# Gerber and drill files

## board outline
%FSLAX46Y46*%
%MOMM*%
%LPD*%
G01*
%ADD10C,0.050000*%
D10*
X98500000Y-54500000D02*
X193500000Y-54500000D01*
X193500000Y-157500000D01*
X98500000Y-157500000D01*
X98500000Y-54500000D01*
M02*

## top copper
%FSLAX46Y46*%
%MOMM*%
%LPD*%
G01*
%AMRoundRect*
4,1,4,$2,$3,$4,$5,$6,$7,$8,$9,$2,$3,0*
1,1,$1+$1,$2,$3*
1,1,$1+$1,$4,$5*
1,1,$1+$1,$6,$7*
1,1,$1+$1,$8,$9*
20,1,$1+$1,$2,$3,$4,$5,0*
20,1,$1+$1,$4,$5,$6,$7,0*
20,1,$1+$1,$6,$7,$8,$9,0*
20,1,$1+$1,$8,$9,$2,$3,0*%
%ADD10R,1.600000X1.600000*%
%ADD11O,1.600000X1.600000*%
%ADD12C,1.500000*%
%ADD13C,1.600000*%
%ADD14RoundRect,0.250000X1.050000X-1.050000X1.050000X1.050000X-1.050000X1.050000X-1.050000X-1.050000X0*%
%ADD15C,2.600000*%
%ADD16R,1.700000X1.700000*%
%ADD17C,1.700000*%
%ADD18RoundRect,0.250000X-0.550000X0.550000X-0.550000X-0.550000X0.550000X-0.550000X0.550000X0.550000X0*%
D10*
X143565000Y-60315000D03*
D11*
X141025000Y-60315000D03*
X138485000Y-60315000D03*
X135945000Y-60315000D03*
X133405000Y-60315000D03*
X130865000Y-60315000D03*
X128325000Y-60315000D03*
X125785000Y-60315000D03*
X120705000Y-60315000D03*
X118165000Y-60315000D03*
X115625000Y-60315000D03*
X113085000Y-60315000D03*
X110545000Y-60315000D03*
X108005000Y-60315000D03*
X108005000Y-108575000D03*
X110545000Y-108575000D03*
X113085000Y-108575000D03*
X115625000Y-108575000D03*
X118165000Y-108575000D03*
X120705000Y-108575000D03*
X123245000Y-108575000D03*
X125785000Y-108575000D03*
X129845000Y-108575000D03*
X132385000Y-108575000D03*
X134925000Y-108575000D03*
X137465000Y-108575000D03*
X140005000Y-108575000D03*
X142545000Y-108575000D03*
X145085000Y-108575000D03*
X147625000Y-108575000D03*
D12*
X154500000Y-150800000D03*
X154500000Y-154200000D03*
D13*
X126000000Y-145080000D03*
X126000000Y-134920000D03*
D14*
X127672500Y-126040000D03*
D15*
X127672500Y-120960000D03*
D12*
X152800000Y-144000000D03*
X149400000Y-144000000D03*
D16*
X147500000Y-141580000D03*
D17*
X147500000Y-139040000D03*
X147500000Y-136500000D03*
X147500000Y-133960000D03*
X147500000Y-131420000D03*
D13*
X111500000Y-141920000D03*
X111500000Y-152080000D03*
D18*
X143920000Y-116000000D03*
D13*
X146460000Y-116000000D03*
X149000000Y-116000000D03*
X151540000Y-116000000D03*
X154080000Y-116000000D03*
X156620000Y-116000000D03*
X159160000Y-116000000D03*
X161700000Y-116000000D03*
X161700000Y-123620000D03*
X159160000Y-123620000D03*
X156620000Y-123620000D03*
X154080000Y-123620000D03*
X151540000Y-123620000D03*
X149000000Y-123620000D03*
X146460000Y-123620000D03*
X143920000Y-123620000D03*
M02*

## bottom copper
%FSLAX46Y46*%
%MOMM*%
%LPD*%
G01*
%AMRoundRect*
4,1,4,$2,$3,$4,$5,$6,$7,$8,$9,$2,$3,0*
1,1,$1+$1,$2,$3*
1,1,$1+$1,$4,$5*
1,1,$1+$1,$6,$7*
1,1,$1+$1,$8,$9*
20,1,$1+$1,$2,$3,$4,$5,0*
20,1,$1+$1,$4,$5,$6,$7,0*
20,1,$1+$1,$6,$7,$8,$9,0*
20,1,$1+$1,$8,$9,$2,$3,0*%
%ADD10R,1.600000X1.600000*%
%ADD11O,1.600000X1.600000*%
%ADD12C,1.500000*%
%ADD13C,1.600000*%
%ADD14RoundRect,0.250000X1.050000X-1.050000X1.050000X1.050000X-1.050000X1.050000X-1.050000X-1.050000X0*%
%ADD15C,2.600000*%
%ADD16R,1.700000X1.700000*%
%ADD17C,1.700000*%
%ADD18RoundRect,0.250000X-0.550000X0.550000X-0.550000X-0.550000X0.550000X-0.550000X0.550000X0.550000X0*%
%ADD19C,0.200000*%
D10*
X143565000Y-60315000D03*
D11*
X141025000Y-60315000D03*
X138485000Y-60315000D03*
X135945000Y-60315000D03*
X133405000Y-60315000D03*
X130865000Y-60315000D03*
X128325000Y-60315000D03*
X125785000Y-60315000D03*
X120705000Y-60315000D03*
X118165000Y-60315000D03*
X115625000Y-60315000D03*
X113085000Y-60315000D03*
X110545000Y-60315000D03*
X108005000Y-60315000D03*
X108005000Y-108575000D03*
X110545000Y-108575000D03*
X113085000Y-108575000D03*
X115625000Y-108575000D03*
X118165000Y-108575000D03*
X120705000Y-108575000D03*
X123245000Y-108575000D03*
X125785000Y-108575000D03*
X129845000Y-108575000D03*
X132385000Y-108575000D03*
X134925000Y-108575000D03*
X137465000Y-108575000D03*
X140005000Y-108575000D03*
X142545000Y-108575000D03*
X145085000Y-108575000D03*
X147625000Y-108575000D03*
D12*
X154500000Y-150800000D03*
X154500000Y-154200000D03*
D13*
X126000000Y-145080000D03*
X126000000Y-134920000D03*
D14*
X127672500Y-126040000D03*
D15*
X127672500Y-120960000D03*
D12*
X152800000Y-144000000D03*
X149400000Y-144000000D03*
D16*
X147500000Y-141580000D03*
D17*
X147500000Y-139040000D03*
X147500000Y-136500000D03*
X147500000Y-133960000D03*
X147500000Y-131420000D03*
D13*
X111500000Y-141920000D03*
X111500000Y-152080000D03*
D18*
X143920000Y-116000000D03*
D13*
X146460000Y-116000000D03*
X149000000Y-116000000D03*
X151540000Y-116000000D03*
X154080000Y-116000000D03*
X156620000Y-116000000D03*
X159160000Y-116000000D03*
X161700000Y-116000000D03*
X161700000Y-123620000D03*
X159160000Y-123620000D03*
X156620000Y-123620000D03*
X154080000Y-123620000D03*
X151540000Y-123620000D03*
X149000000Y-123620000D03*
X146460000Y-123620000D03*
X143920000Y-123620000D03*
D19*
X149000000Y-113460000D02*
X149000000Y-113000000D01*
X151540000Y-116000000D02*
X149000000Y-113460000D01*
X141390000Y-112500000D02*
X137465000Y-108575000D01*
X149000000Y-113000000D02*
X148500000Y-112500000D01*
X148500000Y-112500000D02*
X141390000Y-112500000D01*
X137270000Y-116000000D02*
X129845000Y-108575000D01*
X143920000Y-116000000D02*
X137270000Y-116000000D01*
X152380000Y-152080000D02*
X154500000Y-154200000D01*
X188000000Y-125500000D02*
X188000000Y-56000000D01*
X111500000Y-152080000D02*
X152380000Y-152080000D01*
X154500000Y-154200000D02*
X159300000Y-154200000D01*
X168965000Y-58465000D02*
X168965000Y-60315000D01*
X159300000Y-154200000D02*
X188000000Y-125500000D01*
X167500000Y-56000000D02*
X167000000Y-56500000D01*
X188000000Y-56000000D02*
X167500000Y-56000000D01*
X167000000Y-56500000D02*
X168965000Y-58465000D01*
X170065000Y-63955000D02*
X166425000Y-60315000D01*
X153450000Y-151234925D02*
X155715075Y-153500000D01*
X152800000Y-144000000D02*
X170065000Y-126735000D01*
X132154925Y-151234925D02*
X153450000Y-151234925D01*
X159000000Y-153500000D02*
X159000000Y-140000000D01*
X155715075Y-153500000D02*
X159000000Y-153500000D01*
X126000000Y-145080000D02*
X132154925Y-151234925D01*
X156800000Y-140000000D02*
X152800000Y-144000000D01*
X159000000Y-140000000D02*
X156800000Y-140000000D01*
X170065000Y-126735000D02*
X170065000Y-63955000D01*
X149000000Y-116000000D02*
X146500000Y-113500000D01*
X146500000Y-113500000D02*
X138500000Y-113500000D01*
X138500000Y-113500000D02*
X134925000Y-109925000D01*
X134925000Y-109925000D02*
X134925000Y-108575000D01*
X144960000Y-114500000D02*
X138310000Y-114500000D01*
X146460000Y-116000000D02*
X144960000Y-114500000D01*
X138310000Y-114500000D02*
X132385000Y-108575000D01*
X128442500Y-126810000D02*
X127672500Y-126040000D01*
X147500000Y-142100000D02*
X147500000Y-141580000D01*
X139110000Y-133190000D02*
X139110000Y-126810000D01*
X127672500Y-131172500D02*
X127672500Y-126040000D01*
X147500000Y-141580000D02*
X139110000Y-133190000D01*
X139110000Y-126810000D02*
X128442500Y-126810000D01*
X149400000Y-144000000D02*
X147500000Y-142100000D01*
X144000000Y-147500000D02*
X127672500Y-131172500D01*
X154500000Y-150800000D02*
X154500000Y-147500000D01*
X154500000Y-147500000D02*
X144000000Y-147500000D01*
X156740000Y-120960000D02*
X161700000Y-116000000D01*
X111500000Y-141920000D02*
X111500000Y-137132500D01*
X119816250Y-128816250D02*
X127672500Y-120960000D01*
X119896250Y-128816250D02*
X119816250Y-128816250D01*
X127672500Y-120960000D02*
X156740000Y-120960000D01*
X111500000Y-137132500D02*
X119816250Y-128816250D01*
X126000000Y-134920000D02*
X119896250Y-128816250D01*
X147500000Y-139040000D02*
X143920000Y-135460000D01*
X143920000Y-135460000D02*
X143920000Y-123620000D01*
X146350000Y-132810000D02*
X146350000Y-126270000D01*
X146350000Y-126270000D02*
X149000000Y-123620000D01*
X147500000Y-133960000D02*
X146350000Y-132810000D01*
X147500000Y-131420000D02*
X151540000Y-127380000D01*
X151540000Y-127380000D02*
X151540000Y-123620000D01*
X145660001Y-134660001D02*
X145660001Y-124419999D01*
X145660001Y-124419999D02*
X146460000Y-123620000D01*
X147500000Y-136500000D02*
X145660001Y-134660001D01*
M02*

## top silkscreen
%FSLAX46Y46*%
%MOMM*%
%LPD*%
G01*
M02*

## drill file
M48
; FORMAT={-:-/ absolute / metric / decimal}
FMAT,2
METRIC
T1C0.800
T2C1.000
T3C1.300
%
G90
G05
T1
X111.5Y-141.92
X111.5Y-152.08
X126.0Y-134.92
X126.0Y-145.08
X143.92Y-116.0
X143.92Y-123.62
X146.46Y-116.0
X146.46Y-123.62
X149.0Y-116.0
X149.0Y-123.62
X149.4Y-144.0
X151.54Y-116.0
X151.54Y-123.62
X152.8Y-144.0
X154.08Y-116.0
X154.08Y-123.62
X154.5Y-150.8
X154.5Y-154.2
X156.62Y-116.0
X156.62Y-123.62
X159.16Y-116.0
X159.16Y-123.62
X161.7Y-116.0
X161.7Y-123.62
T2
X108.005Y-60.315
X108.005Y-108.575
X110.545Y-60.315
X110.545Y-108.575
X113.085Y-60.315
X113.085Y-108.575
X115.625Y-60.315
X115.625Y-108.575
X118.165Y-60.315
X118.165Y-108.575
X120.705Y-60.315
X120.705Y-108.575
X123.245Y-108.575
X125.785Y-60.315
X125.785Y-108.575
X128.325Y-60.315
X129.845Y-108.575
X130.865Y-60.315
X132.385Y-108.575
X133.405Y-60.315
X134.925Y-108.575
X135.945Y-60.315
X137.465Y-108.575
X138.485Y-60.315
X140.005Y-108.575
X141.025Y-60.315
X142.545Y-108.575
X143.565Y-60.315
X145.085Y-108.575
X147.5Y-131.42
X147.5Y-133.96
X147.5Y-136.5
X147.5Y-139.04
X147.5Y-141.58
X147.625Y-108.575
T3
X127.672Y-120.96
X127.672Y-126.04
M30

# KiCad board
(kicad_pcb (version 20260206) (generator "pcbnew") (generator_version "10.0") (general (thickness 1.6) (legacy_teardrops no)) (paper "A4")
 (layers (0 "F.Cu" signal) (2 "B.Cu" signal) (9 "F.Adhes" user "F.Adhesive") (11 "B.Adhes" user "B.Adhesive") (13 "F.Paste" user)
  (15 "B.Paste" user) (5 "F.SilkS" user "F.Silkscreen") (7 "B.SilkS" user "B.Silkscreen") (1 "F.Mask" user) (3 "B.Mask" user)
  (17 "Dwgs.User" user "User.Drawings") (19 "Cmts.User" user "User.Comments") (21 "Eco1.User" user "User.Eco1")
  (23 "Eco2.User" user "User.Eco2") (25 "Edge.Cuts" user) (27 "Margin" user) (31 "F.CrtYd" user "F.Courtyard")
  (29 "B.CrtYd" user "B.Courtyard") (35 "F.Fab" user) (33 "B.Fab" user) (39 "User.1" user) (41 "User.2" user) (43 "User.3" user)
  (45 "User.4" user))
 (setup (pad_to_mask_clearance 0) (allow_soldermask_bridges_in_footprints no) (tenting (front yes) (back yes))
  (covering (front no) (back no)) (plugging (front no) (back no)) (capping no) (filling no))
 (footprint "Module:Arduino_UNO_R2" (layer "B.Cu") (at 143.565 60.315 180)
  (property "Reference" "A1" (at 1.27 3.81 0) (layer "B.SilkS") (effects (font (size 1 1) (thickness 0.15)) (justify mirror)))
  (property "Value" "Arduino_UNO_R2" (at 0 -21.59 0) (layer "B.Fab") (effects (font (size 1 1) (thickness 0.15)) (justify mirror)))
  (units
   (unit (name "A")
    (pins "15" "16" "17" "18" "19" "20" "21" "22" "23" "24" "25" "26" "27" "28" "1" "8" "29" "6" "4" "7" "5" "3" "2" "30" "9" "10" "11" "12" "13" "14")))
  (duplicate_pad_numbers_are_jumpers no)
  (pad "1" thru_hole rect (at 0 0 90) (size 1.6 1.6) (drill 1) (layers "*.Cu" "*.Mask") (remove_unused_layers no)
   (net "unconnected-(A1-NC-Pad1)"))
  (pad "2" thru_hole oval (at 2.54 0 90) (size 1.6 1.6) (drill 1) (layers "*.Cu" "*.Mask") (remove_unused_layers no)
   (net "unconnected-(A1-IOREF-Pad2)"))
  (pad "3" thru_hole oval (at 5.08 0 90) (size 1.6 1.6) (drill 1) (layers "*.Cu" "*.Mask") (remove_unused_layers no)
   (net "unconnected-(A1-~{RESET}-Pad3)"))
  (pad "4" thru_hole oval (at 7.62 0 90) (size 1.6 1.6) (drill 1) (layers "*.Cu" "*.Mask") (remove_unused_layers no)
   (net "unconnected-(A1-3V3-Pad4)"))
  (pad "5" thru_hole oval (at 10.16 0 90) (size 1.6 1.6) (drill 1) (layers "*.Cu" "*.Mask") (remove_unused_layers no)
   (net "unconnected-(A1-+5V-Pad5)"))
  (pad "6" thru_hole oval (at 12.7 0 90) (size 1.6 1.6) (drill 1) (layers "*.Cu" "*.Mask") (remove_unused_layers no)
   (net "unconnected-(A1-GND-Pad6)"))
  (pad "7" thru_hole oval (at 15.24 0 90) (size 1.6 1.6) (drill 1) (layers "*.Cu" "*.Mask") (remove_unused_layers no)
   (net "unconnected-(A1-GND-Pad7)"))
  (pad "8" thru_hole oval (at 17.78 0 90) (size 1.6 1.6) (drill 1) (layers "*.Cu" "*.Mask") (remove_unused_layers no)
   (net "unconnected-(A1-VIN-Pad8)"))
  (pad "9" thru_hole oval (at 22.86 0 90) (size 1.6 1.6) (drill 1) (layers "*.Cu" "*.Mask") (remove_unused_layers no) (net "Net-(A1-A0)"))
  (pad "10" thru_hole oval (at 25.4 0 90) (size 1.6 1.6) (drill 1) (layers "*.Cu" "*.Mask") (remove_unused_layers no) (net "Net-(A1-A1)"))
  (pad "11" thru_hole oval (at 27.94 0 90) (size 1.6 1.6) (drill 1) (layers "*.Cu" "*.Mask") (remove_unused_layers no)
   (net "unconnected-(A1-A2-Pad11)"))
  (pad "12" thru_hole oval (at 30.48 0 90) (size 1.6 1.6) (drill 1) (layers "*.Cu" "*.Mask") (remove_unused_layers no)
   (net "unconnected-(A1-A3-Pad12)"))
  (pad "13" thru_hole oval (at 33.02 0 90) (size 1.6 1.6) (drill 1) (layers "*.Cu" "*.Mask") (remove_unused_layers no)
   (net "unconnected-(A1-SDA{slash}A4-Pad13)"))
  (pad "14" thru_hole oval (at 35.56 0 90) (size 1.6 1.6) (drill 1) (layers "*.Cu" "*.Mask") (remove_unused_layers no)
   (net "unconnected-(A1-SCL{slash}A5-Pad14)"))
  (pad "15" thru_hole oval (at 35.56 -48.26 90) (size 1.6 1.6) (drill 1) (layers "*.Cu" "*.Mask") (remove_unused_layers no)
   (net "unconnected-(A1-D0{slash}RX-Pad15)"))
  (pad "16" thru_hole oval (at 33.02 -48.26 90) (size 1.6 1.6) (drill 1) (layers "*.Cu" "*.Mask") (remove_unused_layers no)
   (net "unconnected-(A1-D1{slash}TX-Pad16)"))
  (pad "17" thru_hole oval (at 30.48 -48.26 90) (size 1.6 1.6) (drill 1) (layers "*.Cu" "*.Mask") (remove_unused_layers no)
   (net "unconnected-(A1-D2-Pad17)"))
  (pad "18" thru_hole oval (at 27.94 -48.26 90) (size 1.6 1.6) (drill 1) (layers "*.Cu" "*.Mask") (remove_unused_layers no)
   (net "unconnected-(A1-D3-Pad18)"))
  (pad "19" thru_hole oval (at 25.4 -48.26 90) (size 1.6 1.6) (drill 1) (layers "*.Cu" "*.Mask") (remove_unused_layers no)
   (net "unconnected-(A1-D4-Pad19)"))
  (pad "20" thru_hole oval (at 22.86 -48.26 90) (size 1.6 1.6) (drill 1) (layers "*.Cu" "*.Mask") (remove_unused_layers no)
   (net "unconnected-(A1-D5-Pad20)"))
  (pad "21" thru_hole oval (at 20.32 -48.26 90) (size 1.6 1.6) (drill 1) (layers "*.Cu" "*.Mask") (remove_unused_layers no)
   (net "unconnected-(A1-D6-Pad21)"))
  (pad "22" thru_hole oval (at 17.78 -48.26 90) (size 1.6 1.6) (drill 1) (layers "*.Cu" "*.Mask") (remove_unused_layers no)
   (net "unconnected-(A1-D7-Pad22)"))
  (pad "23" thru_hole oval (at 13.72 -48.26 90) (size 1.6 1.6) (drill 1) (layers "*.Cu" "*.Mask") (remove_unused_layers no)
   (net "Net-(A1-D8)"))
  (pad "24" thru_hole oval (at 11.18 -48.26 90) (size 1.6 1.6) (drill 1) (layers "*.Cu" "*.Mask") (remove_unused_layers no)
   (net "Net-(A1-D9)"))
  (pad "25" thru_hole oval (at 8.64 -48.26 90) (size 1.6 1.6) (drill 1) (layers "*.Cu" "*.Mask") (remove_unused_layers no)
   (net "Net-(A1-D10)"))
  (pad "26" thru_hole oval (at 6.1 -48.26 90) (size 1.6 1.6) (drill 1) (layers "*.Cu" "*.Mask") (remove_unused_layers no)
   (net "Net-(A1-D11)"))
  (pad "27" thru_hole oval (at 3.56 -48.26 90) (size 1.6 1.6) (drill 1) (layers "*.Cu" "*.Mask") (remove_unused_layers no)
   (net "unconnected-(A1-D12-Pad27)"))
  (pad "28" thru_hole oval (at 1.02 -48.26 90) (size 1.6 1.6) (drill 1) (layers "*.Cu" "*.Mask") (remove_unused_layers no)
   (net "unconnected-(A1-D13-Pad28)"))
  (pad "29" thru_hole oval (at -1.52 -48.26 90) (size 1.6 1.6) (drill 1) (layers "*.Cu" "*.Mask") (remove_unused_layers no)
   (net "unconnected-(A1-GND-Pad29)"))
  (pad "30" thru_hole oval (at -4.06 -48.26 90) (size 1.6 1.6) (drill 1) (layers "*.Cu" "*.Mask") (remove_unused_layers no)
   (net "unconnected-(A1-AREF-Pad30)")))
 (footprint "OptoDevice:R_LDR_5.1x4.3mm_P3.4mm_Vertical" (layer "B.Cu") (at 154.5 150.8 -90)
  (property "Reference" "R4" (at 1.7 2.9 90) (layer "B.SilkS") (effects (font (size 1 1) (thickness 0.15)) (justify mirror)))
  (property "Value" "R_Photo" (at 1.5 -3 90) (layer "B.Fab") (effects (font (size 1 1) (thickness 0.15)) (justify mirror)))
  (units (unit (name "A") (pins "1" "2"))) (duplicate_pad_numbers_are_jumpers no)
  (pad "1" thru_hole circle (at 0 0 270) (size 1.5 1.5) (drill 0.8) (layers "*.Cu" "*.Mask") (remove_unused_layers no) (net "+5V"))
  (pad "2" thru_hole circle (at 3.4 0 270) (size 1.5 1.5) (drill 0.8) (layers "*.Cu" "*.Mask") (remove_unused_layers no) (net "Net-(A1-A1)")))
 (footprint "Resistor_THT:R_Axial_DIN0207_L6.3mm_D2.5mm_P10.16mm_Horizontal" (layer "B.Cu") (at 126 145.08 90)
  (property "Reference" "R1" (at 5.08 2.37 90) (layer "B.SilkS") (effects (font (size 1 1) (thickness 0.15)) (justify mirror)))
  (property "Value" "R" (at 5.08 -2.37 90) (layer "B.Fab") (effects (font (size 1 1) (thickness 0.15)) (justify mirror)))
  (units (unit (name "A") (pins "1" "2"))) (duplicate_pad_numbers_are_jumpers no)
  (pad "1" thru_hole circle (at 0 0 90) (size 1.6 1.6) (drill 0.8) (layers "*.Cu" "*.Mask") (remove_unused_layers no) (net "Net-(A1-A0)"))
  (pad "2" thru_hole circle (at 10.16 0 90) (size 1.6 1.6) (drill 0.8) (layers "*.Cu" "*.Mask") (remove_unused_layers no) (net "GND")))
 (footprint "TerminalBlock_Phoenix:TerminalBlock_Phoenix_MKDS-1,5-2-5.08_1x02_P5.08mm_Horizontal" (layer "B.Cu") (at 127.6725 126.04 90)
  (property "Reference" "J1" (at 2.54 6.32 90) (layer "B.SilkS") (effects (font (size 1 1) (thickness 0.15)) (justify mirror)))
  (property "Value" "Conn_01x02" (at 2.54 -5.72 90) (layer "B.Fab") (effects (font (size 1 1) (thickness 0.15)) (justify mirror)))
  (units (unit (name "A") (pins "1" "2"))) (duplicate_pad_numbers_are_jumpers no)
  (pad "1" thru_hole roundrect (at 0 0 90) (size 2.6 2.6) (drill 1.3) (layers "*.Cu" "*.Mask") (remove_unused_layers no)
   (roundrect_rratio 0.096154) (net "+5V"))
  (pad "2" thru_hole circle (at 5.08 0 90) (size 2.6 2.6) (drill 1.3) (layers "*.Cu" "*.Mask") (remove_unused_layers no) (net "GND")))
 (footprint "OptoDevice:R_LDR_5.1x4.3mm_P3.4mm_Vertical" (layer "B.Cu") (at 152.8 144 180)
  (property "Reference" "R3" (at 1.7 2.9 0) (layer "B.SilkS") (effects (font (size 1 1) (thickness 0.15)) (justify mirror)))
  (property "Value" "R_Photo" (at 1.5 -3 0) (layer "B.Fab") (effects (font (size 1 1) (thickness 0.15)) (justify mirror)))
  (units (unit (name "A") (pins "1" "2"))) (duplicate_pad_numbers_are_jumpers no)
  (pad "1" thru_hole circle (at 0 0 180) (size 1.5 1.5) (drill 0.8) (layers "*.Cu" "*.Mask") (remove_unused_layers no) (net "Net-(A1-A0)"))
  (pad "2" thru_hole circle (at 3.4 0 180) (size 1.5 1.5) (drill 0.8) (layers "*.Cu" "*.Mask") (remove_unused_layers no) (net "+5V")))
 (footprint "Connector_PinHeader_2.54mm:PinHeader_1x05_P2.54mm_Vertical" (layer "B.Cu") (at 147.5 141.58)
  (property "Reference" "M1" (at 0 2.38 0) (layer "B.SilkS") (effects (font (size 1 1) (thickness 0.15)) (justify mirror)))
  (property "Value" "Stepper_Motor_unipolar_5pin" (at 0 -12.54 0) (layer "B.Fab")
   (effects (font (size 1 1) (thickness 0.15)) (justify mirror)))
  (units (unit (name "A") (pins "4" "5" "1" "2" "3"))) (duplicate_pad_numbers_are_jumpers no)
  (pad "1" thru_hole rect (at 0 0) (size 1.7 1.7) (drill 1) (layers "*.Cu" "*.Mask") (remove_unused_layers no) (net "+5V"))
  (pad "2" thru_hole circle (at 0 -2.54) (size 1.7 1.7) (drill 1) (layers "*.Cu" "*.Mask") (remove_unused_layers no) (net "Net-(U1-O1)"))
  (pad "3" thru_hole circle (at 0 -5.08) (size 1.7 1.7) (drill 1) (layers "*.Cu" "*.Mask") (remove_unused_layers no) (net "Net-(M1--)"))
  (pad "4" thru_hole circle (at 0 -7.62) (size 1.7 1.7) (drill 1) (layers "*.Cu" "*.Mask") (remove_unused_layers no) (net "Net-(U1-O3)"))
  (pad "5" thru_hole circle (at 0 -10.16) (size 1.7 1.7) (drill 1) (layers "*.Cu" "*.Mask") (remove_unused_layers no) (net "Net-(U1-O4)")))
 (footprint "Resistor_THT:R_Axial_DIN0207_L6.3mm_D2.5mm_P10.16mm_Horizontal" (layer "B.Cu") (at 111.5 141.92 -90)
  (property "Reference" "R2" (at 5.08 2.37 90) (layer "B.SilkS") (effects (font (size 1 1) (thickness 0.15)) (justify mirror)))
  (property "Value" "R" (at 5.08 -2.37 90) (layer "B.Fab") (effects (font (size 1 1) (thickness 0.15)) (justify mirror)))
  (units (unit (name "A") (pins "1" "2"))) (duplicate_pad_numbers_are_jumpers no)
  (pad "1" thru_hole circle (at 0 0 270) (size 1.6 1.6) (drill 0.8) (layers "*.Cu" "*.Mask") (remove_unused_layers no) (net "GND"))
  (pad "2" thru_hole circle (at 10.16 0 270) (size 1.6 1.6) (drill 0.8) (layers "*.Cu" "*.Mask") (remove_unused_layers no)
   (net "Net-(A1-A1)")))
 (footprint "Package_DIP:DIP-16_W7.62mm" (layer "B.Cu") (at 143.92 116 -90)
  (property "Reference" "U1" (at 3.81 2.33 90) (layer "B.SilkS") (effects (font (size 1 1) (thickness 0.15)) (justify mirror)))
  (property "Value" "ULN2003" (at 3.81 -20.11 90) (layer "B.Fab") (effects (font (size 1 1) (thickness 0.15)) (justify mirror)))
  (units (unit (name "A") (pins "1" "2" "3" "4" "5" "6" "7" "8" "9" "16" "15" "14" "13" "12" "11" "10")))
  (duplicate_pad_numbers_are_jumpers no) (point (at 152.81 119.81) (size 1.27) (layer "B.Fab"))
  (pad "1" thru_hole roundrect (at 0 0 270) (size 1.6 1.6) (drill 0.8) (layers "*.Cu" "*.Mask") (remove_unused_layers no)
   (roundrect_rratio 0.15625) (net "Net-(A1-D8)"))
  (pad "2" thru_hole circle (at 0 -2.54 270) (size 1.6 1.6) (drill 0.8) (layers "*.Cu" "*.Mask") (remove_unused_layers no)
   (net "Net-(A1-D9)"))
  (pad "3" thru_hole circle (at 0 -5.08 270) (size 1.6 1.6) (drill 0.8) (layers "*.Cu" "*.Mask") (remove_unused_layers no)
   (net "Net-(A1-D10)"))
  (pad "4" thru_hole circle (at 0 -7.62 270) (size 1.6 1.6) (drill 0.8) (layers "*.Cu" "*.Mask") (remove_unused_layers no)
   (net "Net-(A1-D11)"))
  (pad "5" thru_hole circle (at 0 -10.16 270) (size 1.6 1.6) (drill 0.8) (layers "*.Cu" "*.Mask") (remove_unused_layers no)
   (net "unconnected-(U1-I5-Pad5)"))
  (pad "6" thru_hole circle (at 0 -12.7 270) (size 1.6 1.6) (drill 0.8) (layers "*.Cu" "*.Mask") (remove_unused_layers no)
   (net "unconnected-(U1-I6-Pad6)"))
  (pad "7" thru_hole circle (at 0 -15.24 270) (size 1.6 1.6) (drill 0.8) (layers "*.Cu" "*.Mask") (remove_unused_layers no)
   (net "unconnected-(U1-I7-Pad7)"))
  (pad "8" thru_hole circle (at 0 -17.78 270) (size 1.6 1.6) (drill 0.8) (layers "*.Cu" "*.Mask") (remove_unused_layers no) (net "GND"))
  (pad "9" thru_hole circle (at 7.62 -17.78 270) (size 1.6 1.6) (drill 0.8) (layers "*.Cu" "*.Mask") (remove_unused_layers no) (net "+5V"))
  (pad "10" thru_hole circle (at 7.62 -15.24 270) (size 1.6 1.6) (drill 0.8) (layers "*.Cu" "*.Mask") (remove_unused_layers no)
   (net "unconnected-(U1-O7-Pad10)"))
  (pad "11" thru_hole circle (at 7.62 -12.7 270) (size 1.6 1.6) (drill 0.8) (layers "*.Cu" "*.Mask") (remove_unused_layers no)
   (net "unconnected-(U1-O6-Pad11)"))
  (pad "12" thru_hole circle (at 7.62 -10.16 270) (size 1.6 1.6) (drill 0.8) (layers "*.Cu" "*.Mask") (remove_unused_layers no)
   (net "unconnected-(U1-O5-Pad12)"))
  (pad "13" thru_hole circle (at 7.62 -7.62 270) (size 1.6 1.6) (drill 0.8) (layers "*.Cu" "*.Mask") (remove_unused_layers no)
   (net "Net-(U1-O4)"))
  (pad "14" thru_hole circle (at 7.62 -5.08 270) (size 1.6 1.6) (drill 0.8) (layers "*.Cu" "*.Mask") (remove_unused_layers no)
   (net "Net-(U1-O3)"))
  (pad "15" thru_hole circle (at 7.62 -2.54 270) (size 1.6 1.6) (drill 0.8) (layers "*.Cu" "*.Mask") (remove_unused_layers no)
   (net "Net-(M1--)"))
  (pad "16" thru_hole circle (at 7.62 0 270) (size 1.6 1.6) (drill 0.8) (layers "*.Cu" "*.Mask") (remove_unused_layers no)
   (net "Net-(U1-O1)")))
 (gr_rect (start 98.5 54.5) (end 193.5 157.5) (stroke (width 0.05) (type default)) (fill no) (layer "Edge.Cuts"))
 (segment (start 149 113.46) (end 149 113) (width 0.2) (layer "B.Cu") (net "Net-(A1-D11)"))
 (segment (start 151.54 116) (end 149 113.46) (width 0.2) (layer "B.Cu") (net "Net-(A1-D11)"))
 (segment (start 141.39 112.5) (end 137.465 108.575) (width 0.2) (layer "B.Cu") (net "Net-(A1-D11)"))
 (segment (start 149 113) (end 148.5 112.5) (width 0.2) (layer "B.Cu") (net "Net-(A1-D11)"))
 (segment (start 148.5 112.5) (end 141.39 112.5) (width 0.2) (layer "B.Cu") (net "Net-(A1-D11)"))
 (segment (start 137.27 116) (end 129.845 108.575) (width 0.2) (layer "B.Cu") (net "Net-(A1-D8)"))
 (segment (start 143.92 116) (end 137.27 116) (width 0.2) (layer "B.Cu") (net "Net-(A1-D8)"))
 (segment (start 152.38 152.08) (end 154.5 154.2) (width 0.2) (layer "B.Cu") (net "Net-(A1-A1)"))
 (segment (start 188 125.5) (end 188 56) (width 0.2) (layer "B.Cu") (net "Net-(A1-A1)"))
 (segment (start 111.5 152.08) (end 152.38 152.08) (width 0.2) (layer "B.Cu") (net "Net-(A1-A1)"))
 (segment (start 154.5 154.2) (end 159.3 154.2) (width 0.2) (layer "B.Cu") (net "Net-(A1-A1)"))
 (segment (start 168.965 58.465) (end 168.965 60.315) (width 0.2) (layer "B.Cu") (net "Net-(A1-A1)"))
 (segment (start 159.3 154.2) (end 188 125.5) (width 0.2) (layer "B.Cu") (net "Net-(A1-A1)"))
 (segment (start 167.5 56) (end 167 56.5) (width 0.2) (layer "B.Cu") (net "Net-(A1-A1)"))
 (segment (start 188 56) (end 167.5 56) (width 0.2) (layer "B.Cu") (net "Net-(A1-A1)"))
 (segment (start 167 56.5) (end 168.965 58.465) (width 0.2) (layer "B.Cu") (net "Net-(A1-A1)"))
 (segment (start 170.065 63.955) (end 166.425 60.315) (width 0.2) (layer "B.Cu") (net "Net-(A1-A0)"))
 (segment (start 153.45 151.234925) (end 155.715075 153.5) (width 0.2) (layer "B.Cu") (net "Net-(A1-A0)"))
 (segment (start 152.8 144) (end 170.065 126.735) (width 0.2) (layer "B.Cu") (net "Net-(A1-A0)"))
 (segment (start 132.154925 151.234925) (end 153.45 151.234925) (width 0.2) (layer "B.Cu") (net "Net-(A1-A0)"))
 (segment (start 159 153.5) (end 159 140) (width 0.2) (layer "B.Cu") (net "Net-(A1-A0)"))
 (segment (start 155.715075 153.5) (end 159 153.5) (width 0.2) (layer "B.Cu") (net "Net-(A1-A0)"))
 (segment (start 126 145.08) (end 132.154925 151.234925) (width 0.2) (layer "B.Cu") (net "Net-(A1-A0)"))
 (segment (start 156.8 140) (end 152.8 144) (width 0.2) (layer "B.Cu") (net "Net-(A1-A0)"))
 (segment (start 159 140) (end 156.8 140) (width 0.2) (layer "B.Cu") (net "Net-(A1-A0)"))
 (segment (start 170.065 126.735) (end 170.065 63.955) (width 0.2) (layer "B.Cu") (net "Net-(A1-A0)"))
 (segment (start 149 116) (end 146.5 113.5) (width 0.2) (layer "B.Cu") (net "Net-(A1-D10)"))
 (segment (start 146.5 113.5) (end 138.5 113.5) (width 0.2) (layer "B.Cu") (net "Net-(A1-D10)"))
 (segment (start 138.5 113.5) (end 134.925 109.925) (width 0.2) (layer "B.Cu") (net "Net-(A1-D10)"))
 (segment (start 134.925 109.925) (end 134.925 108.575) (width 0.2) (layer "B.Cu") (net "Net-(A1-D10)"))
 (segment (start 144.96 114.5) (end 138.31 114.5) (width 0.2) (layer "B.Cu") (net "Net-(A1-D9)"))
 (segment (start 146.46 116) (end 144.96 114.5) (width 0.2) (layer "B.Cu") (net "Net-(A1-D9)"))
 (segment (start 138.31 114.5) (end 132.385 108.575) (width 0.2) (layer "B.Cu") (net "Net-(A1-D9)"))
 (segment (start 128.4425 126.81) (end 127.6725 126.04) (width 0.2) (layer "B.Cu") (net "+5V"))
 (segment (start 147.5 142.1) (end 147.5 141.58) (width 0.2) (layer "B.Cu") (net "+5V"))
 (segment (start 139.11 133.19) (end 139.11 126.81) (width 0.2) (layer "B.Cu") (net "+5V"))
 (segment (start 127.6725 131.1725) (end 127.6725 126.04) (width 0.2) (layer "B.Cu") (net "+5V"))
 (segment (start 147.5 141.58) (end 139.11 133.19) (width 0.2) (layer "B.Cu") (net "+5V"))
 (segment (start 139.11 126.81) (end 128.4425 126.81) (width 0.2) (layer "B.Cu") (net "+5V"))
 (segment (start 149.4 144) (end 147.5 142.1) (width 0.2) (layer "B.Cu") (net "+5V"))
 (segment (start 144 147.5) (end 127.6725 131.1725) (width 0.2) (layer "B.Cu") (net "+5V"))
 (segment (start 154.5 150.8) (end 154.5 147.5) (width 0.2) (layer "B.Cu") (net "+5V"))
 (segment (start 154.5 147.5) (end 144 147.5) (width 0.2) (layer "B.Cu") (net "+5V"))
 (segment (start 156.74 120.96) (end 161.7 116) (width 0.2) (layer "B.Cu") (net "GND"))
 (segment (start 111.5 141.92) (end 111.5 137.1325) (width 0.2) (layer "B.Cu") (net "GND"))
 (segment (start 119.81625 128.81625) (end 127.6725 120.96) (width 0.2) (layer "B.Cu") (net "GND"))
 (segment (start 119.89625 128.81625) (end 119.81625 128.81625) (width 0.2) (layer "B.Cu") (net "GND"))
 (segment (start 127.6725 120.96) (end 156.74 120.96) (width 0.2) (layer "B.Cu") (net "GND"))
 (segment (start 111.5 137.1325) (end 119.81625 128.81625) (width 0.2) (layer "B.Cu") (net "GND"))
 (segment (start 126 134.92) (end 119.89625 128.81625) (width 0.2) (layer "B.Cu") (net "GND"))
 (segment (start 147.5 139.04) (end 143.92 135.46) (width 0.2) (layer "B.Cu") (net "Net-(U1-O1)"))
 (segment (start 143.92 135.46) (end 143.92 123.62) (width 0.2) (layer "B.Cu") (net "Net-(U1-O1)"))
 (segment (start 146.35 132.81) (end 146.35 126.27) (width 0.2) (layer "B.Cu") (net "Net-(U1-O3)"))
 (segment (start 146.35 126.27) (end 149 123.62) (width 0.2) (layer "B.Cu") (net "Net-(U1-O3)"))
 (segment (start 147.5 133.96) (end 146.35 132.81) (width 0.2) (layer "B.Cu") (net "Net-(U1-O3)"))
 (segment (start 147.5 131.42) (end 151.54 127.38) (width 0.2) (layer "B.Cu") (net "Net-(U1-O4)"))
 (segment (start 151.54 127.38) (end 151.54 123.62) (width 0.2) (layer "B.Cu") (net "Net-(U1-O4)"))
 (segment (start 145.660001 134.660001) (end 145.660001 124.419999) (width 0.2) (layer "B.Cu") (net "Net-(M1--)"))
 (segment (start 145.660001 124.419999) (end 146.46 123.62) (width 0.2) (layer "B.Cu") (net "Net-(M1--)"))
 (segment (start 147.5 136.5) (end 145.660001 134.660001) (width 0.2) (layer "B.Cu") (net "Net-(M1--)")))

